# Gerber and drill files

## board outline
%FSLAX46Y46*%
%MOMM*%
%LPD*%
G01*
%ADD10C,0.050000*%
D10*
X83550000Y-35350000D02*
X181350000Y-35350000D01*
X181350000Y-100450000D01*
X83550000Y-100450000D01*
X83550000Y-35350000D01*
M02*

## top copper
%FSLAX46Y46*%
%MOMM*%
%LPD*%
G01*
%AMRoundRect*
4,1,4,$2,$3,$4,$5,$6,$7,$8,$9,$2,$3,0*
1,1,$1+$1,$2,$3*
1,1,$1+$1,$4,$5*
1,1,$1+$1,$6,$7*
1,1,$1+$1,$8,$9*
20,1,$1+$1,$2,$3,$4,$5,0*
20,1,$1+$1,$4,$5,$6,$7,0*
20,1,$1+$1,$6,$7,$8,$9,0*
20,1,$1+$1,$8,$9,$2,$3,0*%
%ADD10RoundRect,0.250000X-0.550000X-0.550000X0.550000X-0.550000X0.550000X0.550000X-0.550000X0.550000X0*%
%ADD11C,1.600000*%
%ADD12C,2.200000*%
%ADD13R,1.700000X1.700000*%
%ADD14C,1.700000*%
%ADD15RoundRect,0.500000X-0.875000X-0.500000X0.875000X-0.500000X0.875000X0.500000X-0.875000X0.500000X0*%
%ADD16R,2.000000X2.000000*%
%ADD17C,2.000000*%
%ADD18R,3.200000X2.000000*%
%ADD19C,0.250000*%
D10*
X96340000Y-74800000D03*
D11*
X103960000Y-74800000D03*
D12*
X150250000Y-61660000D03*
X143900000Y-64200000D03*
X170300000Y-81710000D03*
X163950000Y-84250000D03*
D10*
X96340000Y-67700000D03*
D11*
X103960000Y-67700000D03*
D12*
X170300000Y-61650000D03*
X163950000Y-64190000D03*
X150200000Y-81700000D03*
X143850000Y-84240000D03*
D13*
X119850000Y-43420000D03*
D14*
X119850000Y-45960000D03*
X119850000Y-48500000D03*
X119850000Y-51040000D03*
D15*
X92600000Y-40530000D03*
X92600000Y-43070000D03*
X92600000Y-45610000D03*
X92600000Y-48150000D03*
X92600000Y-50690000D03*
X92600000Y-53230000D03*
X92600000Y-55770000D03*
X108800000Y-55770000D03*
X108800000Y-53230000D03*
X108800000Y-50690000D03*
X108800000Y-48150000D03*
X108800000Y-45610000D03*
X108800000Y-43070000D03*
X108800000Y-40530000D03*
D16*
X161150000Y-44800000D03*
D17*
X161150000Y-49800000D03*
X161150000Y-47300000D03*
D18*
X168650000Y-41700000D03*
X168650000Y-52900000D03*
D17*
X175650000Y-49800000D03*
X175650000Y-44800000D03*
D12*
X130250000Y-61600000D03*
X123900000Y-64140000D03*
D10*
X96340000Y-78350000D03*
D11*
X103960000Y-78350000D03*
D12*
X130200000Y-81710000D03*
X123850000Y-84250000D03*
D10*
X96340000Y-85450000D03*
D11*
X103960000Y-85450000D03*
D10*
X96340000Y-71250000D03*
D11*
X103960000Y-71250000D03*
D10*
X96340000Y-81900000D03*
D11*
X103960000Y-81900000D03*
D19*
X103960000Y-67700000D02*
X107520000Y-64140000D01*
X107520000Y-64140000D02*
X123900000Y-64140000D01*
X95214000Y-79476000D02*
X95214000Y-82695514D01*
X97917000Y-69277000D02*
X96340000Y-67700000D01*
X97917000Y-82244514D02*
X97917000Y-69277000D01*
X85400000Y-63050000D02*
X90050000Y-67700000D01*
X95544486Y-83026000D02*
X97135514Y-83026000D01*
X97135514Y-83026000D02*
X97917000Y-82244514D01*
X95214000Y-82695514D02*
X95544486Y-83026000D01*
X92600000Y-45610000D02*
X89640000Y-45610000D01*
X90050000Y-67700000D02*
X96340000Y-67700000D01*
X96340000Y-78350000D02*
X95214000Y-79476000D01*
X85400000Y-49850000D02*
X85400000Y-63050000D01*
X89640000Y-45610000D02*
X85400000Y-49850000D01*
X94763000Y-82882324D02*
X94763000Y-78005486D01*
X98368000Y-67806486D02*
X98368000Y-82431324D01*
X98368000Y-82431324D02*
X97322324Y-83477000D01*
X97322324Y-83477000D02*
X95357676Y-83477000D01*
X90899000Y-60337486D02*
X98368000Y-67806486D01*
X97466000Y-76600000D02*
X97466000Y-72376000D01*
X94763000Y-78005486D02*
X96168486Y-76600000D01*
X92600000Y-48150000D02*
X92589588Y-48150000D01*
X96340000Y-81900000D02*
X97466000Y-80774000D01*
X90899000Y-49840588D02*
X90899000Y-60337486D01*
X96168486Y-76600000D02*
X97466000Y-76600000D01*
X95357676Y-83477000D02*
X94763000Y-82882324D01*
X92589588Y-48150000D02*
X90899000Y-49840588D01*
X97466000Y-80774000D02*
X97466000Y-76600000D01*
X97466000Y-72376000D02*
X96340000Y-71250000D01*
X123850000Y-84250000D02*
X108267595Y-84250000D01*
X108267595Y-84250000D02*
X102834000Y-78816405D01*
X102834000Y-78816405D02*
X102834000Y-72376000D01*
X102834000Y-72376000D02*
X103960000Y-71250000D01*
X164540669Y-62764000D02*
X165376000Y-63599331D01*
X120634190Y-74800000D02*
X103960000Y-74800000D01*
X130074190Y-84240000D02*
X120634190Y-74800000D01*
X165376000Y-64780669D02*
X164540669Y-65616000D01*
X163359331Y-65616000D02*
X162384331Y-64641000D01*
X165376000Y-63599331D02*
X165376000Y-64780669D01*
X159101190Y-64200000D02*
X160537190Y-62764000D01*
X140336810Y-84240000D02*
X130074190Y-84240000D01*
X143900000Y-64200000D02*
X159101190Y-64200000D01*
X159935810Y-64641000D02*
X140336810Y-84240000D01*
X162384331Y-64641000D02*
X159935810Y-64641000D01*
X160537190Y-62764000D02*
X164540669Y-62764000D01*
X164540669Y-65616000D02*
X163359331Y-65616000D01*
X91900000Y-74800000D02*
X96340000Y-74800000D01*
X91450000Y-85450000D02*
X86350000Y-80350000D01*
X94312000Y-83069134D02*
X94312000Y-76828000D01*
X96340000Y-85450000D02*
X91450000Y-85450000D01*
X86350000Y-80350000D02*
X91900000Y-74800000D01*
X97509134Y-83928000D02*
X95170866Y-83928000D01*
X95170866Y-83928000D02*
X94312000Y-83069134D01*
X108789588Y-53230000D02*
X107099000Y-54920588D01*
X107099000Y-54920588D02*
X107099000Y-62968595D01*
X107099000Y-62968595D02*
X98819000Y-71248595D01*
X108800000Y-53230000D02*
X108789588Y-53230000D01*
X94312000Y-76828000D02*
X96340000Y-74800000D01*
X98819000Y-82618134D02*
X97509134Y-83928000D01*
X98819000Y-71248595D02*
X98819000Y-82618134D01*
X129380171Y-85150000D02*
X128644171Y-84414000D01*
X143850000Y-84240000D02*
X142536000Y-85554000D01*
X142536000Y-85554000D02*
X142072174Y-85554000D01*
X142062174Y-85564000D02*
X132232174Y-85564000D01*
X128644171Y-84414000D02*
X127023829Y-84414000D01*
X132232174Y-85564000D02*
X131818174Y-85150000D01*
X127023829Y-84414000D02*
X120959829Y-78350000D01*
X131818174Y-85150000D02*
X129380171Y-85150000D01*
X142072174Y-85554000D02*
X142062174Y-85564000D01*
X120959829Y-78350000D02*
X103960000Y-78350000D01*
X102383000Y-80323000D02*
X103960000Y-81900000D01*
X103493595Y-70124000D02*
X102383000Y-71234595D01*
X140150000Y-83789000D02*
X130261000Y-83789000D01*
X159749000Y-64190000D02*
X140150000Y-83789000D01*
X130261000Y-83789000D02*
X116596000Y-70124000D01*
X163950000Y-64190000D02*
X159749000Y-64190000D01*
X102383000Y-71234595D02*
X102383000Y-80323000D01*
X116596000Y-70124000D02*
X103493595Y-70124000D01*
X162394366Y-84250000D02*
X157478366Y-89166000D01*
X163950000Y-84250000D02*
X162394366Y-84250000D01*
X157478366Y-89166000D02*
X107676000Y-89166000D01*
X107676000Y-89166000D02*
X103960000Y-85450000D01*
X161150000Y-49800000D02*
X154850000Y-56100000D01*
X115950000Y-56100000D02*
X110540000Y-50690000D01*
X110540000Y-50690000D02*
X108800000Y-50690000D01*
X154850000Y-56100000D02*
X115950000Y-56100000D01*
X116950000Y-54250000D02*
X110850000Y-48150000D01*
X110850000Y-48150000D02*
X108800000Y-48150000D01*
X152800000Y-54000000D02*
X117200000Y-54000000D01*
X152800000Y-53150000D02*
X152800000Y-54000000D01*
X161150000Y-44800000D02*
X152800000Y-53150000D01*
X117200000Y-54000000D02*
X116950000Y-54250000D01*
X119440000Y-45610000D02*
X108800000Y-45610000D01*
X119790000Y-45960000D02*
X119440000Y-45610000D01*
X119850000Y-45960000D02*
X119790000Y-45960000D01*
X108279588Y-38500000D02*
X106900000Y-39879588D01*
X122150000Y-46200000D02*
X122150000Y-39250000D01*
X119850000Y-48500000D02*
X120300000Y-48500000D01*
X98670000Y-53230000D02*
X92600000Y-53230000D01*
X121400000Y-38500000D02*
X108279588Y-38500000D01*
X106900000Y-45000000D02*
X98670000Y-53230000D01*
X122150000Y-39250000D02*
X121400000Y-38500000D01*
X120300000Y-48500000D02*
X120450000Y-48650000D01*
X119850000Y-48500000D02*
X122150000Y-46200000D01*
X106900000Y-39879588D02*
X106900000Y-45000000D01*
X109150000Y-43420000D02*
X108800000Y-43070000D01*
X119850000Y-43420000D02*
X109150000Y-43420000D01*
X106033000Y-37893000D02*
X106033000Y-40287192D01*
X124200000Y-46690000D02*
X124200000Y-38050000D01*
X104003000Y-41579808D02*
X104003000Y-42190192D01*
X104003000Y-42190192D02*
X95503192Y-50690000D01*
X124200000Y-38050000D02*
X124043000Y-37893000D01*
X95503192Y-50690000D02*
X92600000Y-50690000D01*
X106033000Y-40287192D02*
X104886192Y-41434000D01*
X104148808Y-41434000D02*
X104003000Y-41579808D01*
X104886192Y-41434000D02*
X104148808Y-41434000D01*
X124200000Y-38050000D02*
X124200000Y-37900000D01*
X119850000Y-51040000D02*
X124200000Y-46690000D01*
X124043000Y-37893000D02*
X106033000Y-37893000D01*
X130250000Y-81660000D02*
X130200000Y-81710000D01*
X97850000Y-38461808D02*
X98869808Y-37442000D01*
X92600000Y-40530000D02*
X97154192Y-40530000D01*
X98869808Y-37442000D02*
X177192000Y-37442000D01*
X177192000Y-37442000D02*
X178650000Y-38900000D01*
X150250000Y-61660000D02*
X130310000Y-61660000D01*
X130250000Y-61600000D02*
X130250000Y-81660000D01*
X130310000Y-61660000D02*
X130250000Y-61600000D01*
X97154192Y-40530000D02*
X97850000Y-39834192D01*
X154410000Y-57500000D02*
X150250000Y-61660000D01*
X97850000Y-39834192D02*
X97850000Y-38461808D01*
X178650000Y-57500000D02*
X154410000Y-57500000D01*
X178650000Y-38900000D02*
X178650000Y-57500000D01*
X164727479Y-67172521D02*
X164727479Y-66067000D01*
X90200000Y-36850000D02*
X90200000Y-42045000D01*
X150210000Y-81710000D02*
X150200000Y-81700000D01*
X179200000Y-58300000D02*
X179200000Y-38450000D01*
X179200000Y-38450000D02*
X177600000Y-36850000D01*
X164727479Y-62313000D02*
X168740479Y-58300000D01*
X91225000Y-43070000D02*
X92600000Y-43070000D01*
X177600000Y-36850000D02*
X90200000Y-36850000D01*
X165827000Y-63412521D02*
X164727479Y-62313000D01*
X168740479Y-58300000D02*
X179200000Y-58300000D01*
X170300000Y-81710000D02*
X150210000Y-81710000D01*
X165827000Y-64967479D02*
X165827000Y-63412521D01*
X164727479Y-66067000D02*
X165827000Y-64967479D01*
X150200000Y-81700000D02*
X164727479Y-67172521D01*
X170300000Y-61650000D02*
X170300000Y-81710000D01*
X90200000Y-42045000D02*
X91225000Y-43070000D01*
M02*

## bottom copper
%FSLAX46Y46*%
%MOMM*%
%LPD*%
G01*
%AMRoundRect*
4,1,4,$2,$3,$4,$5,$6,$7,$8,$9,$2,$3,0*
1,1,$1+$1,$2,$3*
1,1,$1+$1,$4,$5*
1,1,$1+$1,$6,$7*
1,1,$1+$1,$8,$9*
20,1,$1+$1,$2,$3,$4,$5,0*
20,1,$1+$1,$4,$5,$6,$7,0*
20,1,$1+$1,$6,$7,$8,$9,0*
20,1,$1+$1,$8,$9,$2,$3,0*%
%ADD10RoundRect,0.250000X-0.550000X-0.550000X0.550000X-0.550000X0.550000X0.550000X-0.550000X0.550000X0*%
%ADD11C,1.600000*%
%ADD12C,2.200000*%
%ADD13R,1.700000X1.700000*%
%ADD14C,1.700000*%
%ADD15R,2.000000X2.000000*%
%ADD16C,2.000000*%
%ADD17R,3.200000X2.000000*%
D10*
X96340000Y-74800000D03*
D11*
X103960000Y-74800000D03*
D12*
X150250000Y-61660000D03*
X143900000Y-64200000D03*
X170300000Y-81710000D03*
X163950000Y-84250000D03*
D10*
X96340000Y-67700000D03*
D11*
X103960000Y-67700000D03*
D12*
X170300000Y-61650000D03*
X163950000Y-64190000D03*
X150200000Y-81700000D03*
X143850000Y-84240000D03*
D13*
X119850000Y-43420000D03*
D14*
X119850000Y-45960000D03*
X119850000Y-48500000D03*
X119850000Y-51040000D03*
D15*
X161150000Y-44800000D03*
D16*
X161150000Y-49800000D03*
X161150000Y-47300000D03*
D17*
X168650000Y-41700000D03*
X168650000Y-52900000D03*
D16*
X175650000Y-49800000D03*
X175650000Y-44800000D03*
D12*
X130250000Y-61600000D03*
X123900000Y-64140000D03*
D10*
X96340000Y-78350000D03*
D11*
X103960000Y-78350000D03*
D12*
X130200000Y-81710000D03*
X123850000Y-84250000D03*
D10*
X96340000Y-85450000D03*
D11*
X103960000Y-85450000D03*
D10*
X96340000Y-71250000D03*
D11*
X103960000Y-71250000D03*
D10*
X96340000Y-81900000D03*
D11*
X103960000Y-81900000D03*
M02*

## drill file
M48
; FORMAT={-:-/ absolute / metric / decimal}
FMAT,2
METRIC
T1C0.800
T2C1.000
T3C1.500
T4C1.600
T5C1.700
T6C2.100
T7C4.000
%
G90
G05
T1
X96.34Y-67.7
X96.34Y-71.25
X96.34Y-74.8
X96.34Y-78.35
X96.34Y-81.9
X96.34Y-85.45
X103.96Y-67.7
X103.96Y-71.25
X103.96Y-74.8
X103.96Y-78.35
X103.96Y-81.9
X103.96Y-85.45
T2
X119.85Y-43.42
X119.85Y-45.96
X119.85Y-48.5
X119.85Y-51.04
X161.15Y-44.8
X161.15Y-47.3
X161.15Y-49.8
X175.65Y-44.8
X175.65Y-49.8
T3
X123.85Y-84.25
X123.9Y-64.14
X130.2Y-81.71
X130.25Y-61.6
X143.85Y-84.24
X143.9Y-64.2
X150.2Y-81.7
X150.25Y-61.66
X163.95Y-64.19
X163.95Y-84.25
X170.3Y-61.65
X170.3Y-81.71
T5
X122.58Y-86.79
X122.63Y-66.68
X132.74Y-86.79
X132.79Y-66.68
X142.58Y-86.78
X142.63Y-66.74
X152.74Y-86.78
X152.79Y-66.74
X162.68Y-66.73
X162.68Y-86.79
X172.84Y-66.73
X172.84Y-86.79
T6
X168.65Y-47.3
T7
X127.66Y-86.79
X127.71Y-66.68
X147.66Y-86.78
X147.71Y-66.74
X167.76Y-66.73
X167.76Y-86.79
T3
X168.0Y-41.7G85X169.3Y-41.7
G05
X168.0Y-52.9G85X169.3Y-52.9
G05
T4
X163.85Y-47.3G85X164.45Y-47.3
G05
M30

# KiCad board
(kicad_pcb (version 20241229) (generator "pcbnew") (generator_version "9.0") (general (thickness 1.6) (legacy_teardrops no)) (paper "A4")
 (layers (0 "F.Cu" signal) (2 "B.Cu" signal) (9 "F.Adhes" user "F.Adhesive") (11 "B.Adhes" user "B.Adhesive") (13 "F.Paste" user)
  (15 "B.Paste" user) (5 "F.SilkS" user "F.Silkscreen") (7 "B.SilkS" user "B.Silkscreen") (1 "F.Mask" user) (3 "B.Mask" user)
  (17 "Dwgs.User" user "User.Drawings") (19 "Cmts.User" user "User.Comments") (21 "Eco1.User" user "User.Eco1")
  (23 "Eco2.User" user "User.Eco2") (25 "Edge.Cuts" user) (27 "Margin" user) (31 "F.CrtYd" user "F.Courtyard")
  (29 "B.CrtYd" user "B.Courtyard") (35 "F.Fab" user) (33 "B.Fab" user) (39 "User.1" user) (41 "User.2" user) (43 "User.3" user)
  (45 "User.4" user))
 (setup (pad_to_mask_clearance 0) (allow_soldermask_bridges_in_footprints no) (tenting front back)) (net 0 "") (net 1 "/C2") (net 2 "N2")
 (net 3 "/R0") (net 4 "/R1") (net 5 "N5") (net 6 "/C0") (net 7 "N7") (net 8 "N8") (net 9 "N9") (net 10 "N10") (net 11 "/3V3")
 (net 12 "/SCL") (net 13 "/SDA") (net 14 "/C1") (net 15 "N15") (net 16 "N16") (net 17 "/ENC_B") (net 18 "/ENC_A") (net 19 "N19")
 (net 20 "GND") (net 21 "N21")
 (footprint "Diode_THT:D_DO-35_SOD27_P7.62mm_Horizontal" (layer "F.Cu") (at 96.34 74.8)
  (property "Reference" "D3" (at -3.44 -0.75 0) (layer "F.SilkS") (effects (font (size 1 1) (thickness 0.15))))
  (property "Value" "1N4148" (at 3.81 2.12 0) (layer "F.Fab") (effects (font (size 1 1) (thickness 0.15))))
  (pad "1" thru_hole roundrect (at 0 0) (size 1.6 1.6) (drill 0.8) (layers "*.Cu" "*.Mask") (remove_unused_layers no)
   (roundrect_rratio 0.15625) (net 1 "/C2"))
  (pad "2" thru_hole circle (at 7.62 0) (size 1.6 1.6) (drill 0.8) (layers "*.Cu" "*.Mask") (remove_unused_layers no) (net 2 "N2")))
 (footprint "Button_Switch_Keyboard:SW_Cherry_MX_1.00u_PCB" (layer "F.Cu") (at 150.25 61.66)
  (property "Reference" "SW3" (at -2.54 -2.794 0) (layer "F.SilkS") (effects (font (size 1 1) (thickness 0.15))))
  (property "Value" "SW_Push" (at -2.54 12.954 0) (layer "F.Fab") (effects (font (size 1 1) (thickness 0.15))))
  (pad "" np_thru_hole circle (at -7.62 5.08) (size 1.7 1.7) (drill 1.7) (layers "*.Cu" "*.Mask"))
  (pad "" np_thru_hole circle (at -2.54 5.08) (size 4 4) (drill 4) (layers "*.Cu" "*.Mask"))
  (pad "" np_thru_hole circle (at 2.54 5.08) (size 1.7 1.7) (drill 1.7) (layers "*.Cu" "*.Mask"))
  (pad "1" thru_hole circle (at 0 0) (size 2.2 2.2) (drill 1.5) (layers "*.Cu" "*.Mask") (remove_unused_layers no) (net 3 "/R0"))
  (pad "2" thru_hole circle (at -6.35 2.54) (size 2.2 2.2) (drill 1.5) (layers "*.Cu" "*.Mask") (remove_unused_layers no) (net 2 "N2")))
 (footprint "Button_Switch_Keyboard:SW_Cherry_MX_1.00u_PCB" (layer "F.Cu") (at 170.3 81.71)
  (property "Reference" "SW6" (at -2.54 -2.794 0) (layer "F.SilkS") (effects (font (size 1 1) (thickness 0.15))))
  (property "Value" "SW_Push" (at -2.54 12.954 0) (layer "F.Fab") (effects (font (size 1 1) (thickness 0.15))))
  (pad "" np_thru_hole circle (at -7.62 5.08) (size 1.7 1.7) (drill 1.7) (layers "*.Cu" "*.Mask"))
  (pad "" np_thru_hole circle (at -2.54 5.08) (size 4 4) (drill 4) (layers "*.Cu" "*.Mask"))
  (pad "" np_thru_hole circle (at 2.54 5.08) (size 1.7 1.7) (drill 1.7) (layers "*.Cu" "*.Mask"))
  (pad "1" thru_hole circle (at 0 0) (size 2.2 2.2) (drill 1.5) (layers "*.Cu" "*.Mask") (remove_unused_layers no) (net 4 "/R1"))
  (pad "2" thru_hole circle (at -6.35 2.54) (size 2.2 2.2) (drill 1.5) (layers "*.Cu" "*.Mask") (remove_unused_layers no) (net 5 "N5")))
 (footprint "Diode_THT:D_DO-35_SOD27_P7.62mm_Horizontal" (layer "F.Cu") (at 96.34 67.7)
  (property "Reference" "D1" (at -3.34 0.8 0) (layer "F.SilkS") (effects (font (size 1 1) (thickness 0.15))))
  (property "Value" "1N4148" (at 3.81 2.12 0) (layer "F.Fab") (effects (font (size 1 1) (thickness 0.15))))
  (pad "1" thru_hole roundrect (at 0 0) (size 1.6 1.6) (drill 0.8) (layers "*.Cu" "*.Mask") (remove_unused_layers no)
   (roundrect_rratio 0.15625) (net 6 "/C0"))
  (pad "2" thru_hole circle (at 7.62 0) (size 1.6 1.6) (drill 0.8) (layers "*.Cu" "*.Mask") (remove_unused_layers no) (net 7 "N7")))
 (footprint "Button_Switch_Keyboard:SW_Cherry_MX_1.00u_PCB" (layer "F.Cu") (at 170.3 61.65)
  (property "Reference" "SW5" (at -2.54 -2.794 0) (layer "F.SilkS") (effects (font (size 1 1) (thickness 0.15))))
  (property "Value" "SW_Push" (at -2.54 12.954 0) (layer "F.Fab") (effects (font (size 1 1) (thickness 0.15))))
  (pad "" np_thru_hole circle (at -7.62 5.08) (size 1.7 1.7) (drill 1.7) (layers "*.Cu" "*.Mask"))
  (pad "" np_thru_hole circle (at -2.54 5.08) (size 4 4) (drill 4) (layers "*.Cu" "*.Mask"))
  (pad "" np_thru_hole circle (at 2.54 5.08) (size 1.7 1.7) (drill 1.7) (layers "*.Cu" "*.Mask"))
  (pad "1" thru_hole circle (at 0 0) (size 2.2 2.2) (drill 1.5) (layers "*.Cu" "*.Mask") (remove_unused_layers no) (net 4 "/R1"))
  (pad "2" thru_hole circle (at -6.35 2.54) (size 2.2 2.2) (drill 1.5) (layers "*.Cu" "*.Mask") (remove_unused_layers no) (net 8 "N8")))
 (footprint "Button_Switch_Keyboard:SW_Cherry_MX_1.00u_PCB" (layer "F.Cu") (at 150.2 81.7)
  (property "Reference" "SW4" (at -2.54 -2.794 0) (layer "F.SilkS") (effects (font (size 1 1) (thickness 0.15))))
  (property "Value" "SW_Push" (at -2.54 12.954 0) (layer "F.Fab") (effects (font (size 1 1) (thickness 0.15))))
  (pad "" np_thru_hole circle (at -7.62 5.08) (size 1.7 1.7) (drill 1.7) (layers "*.Cu" "*.Mask"))
  (pad "" np_thru_hole circle (at -2.54 5.08) (size 4 4) (drill 4) (layers "*.Cu" "*.Mask"))
  (pad "" np_thru_hole circle (at 2.54 5.08) (size 1.7 1.7) (drill 1.7) (layers "*.Cu" "*.Mask"))
  (pad "1" thru_hole circle (at 0 0) (size 2.2 2.2) (drill 1.5) (layers "*.Cu" "*.Mask") (remove_unused_layers no) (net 4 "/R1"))
  (pad "2" thru_hole circle (at -6.35 2.54) (size 2.2 2.2) (drill 1.5) (layers "*.Cu" "*.Mask") (remove_unused_layers no) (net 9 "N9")))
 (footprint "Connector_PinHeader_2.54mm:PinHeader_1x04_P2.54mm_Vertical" (layer "F.Cu") (at 119.85 43.42)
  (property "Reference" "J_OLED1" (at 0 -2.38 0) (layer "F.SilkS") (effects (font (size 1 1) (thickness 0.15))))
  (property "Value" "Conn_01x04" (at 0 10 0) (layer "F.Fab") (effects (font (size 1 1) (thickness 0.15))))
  (pad "1" thru_hole rect (at 0 0) (size 1.7 1.7) (drill 1) (layers "*.Cu" "*.Mask") (remove_unused_layers no) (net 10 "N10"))
  (pad "2" thru_hole circle (at 0 2.54) (size 1.7 1.7) (drill 1) (layers "*.Cu" "*.Mask") (remove_unused_layers no) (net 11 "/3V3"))
  (pad "3" thru_hole circle (at 0 5.08) (size 1.7 1.7) (drill 1) (layers "*.Cu" "*.Mask") (remove_unused_layers no) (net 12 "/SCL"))
  (pad "4" thru_hole circle (at 0 7.62) (size 1.7 1.7) (drill 1) (layers "*.Cu" "*.Mask") (remove_unused_layers no) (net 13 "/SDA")))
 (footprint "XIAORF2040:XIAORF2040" (layer "F.Cu") (at 100.7 48.15)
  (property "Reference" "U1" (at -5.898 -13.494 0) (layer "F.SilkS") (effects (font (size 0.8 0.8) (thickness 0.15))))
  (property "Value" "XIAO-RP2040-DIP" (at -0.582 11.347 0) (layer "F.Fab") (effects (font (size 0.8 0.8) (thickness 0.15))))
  (pad "1" smd roundrect (at -8.1 -7.62) (size 2.75 2) (layers "F.Cu" "F.Mask" "F.Paste") (roundrect_rratio 0.25) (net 3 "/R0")
   (solder_mask_margin 0.102))
  (pad "2" smd roundrect (at -8.1 -5.08) (size 2.75 2) (layers "F.Cu" "F.Mask" "F.Paste") (roundrect_rratio 0.25) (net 4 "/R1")
   (solder_mask_margin 0.102))
  (pad "3" smd roundrect (at -8.1 -2.54) (size 2.75 2) (layers "F.Cu" "F.Mask" "F.Paste") (roundrect_rratio 0.25) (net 6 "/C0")
   (solder_mask_margin 0.102))
  (pad "4" smd roundrect (at -8.1 0) (size 2.75 2) (layers "F.Cu" "F.Mask" "F.Paste") (roundrect_rratio 0.25) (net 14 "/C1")
   (solder_mask_margin 0.102))
  (pad "5" smd roundrect (at -8.1 2.54) (size 2.75 2) (layers "F.Cu" "F.Mask" "F.Paste") (roundrect_rratio 0.25) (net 13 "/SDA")
   (solder_mask_margin 0.102))
  (pad "6" smd roundrect (at -8.1 5.08) (size 2.75 2) (layers "F.Cu" "F.Mask" "F.Paste") (roundrect_rratio 0.25) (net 12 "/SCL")
   (solder_mask_margin 0.102))
  (pad "7" smd roundrect (at -8.1 7.62) (size 2.75 2) (layers "F.Cu" "F.Mask" "F.Paste") (roundrect_rratio 0.25) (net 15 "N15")
   (solder_mask_margin 0.102))
  (pad "8" smd roundrect (at 8.1 7.62) (size 2.75 2) (layers "F.Cu" "F.Mask" "F.Paste") (roundrect_rratio 0.25) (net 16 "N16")
   (solder_mask_margin 0.102))
  (pad "9" smd roundrect (at 8.1 5.08) (size 2.75 2) (layers "F.Cu" "F.Mask" "F.Paste") (roundrect_rratio 0.25) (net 1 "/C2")
   (solder_mask_margin 0.102))
  (pad "10" smd roundrect (at 8.1 2.54) (size 2.75 2) (layers "F.Cu" "F.Mask" "F.Paste") (roundrect_rratio 0.25) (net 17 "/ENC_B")
   (solder_mask_margin 0.102))
  (pad "11" smd roundrect (at 8.1 0) (size 2.75 2) (layers "F.Cu" "F.Mask" "F.Paste") (roundrect_rratio 0.25) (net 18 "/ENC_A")
   (solder_mask_margin 0.102))
  (pad "12" smd roundrect (at 8.1 -2.54) (size 2.75 2) (layers "F.Cu" "F.Mask" "F.Paste") (roundrect_rratio 0.25) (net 11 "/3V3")
   (solder_mask_margin 0.102))
  (pad "13" smd roundrect (at 8.1 -5.08) (size 2.75 2) (layers "F.Cu" "F.Mask" "F.Paste") (roundrect_rratio 0.25) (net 10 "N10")
   (solder_mask_margin 0.102))
  (pad "14" smd roundrect (at 8.1 -7.62) (size 2.75 2) (layers "F.Cu" "F.Mask" "F.Paste") (roundrect_rratio 0.25) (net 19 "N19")
   (solder_mask_margin 0.102))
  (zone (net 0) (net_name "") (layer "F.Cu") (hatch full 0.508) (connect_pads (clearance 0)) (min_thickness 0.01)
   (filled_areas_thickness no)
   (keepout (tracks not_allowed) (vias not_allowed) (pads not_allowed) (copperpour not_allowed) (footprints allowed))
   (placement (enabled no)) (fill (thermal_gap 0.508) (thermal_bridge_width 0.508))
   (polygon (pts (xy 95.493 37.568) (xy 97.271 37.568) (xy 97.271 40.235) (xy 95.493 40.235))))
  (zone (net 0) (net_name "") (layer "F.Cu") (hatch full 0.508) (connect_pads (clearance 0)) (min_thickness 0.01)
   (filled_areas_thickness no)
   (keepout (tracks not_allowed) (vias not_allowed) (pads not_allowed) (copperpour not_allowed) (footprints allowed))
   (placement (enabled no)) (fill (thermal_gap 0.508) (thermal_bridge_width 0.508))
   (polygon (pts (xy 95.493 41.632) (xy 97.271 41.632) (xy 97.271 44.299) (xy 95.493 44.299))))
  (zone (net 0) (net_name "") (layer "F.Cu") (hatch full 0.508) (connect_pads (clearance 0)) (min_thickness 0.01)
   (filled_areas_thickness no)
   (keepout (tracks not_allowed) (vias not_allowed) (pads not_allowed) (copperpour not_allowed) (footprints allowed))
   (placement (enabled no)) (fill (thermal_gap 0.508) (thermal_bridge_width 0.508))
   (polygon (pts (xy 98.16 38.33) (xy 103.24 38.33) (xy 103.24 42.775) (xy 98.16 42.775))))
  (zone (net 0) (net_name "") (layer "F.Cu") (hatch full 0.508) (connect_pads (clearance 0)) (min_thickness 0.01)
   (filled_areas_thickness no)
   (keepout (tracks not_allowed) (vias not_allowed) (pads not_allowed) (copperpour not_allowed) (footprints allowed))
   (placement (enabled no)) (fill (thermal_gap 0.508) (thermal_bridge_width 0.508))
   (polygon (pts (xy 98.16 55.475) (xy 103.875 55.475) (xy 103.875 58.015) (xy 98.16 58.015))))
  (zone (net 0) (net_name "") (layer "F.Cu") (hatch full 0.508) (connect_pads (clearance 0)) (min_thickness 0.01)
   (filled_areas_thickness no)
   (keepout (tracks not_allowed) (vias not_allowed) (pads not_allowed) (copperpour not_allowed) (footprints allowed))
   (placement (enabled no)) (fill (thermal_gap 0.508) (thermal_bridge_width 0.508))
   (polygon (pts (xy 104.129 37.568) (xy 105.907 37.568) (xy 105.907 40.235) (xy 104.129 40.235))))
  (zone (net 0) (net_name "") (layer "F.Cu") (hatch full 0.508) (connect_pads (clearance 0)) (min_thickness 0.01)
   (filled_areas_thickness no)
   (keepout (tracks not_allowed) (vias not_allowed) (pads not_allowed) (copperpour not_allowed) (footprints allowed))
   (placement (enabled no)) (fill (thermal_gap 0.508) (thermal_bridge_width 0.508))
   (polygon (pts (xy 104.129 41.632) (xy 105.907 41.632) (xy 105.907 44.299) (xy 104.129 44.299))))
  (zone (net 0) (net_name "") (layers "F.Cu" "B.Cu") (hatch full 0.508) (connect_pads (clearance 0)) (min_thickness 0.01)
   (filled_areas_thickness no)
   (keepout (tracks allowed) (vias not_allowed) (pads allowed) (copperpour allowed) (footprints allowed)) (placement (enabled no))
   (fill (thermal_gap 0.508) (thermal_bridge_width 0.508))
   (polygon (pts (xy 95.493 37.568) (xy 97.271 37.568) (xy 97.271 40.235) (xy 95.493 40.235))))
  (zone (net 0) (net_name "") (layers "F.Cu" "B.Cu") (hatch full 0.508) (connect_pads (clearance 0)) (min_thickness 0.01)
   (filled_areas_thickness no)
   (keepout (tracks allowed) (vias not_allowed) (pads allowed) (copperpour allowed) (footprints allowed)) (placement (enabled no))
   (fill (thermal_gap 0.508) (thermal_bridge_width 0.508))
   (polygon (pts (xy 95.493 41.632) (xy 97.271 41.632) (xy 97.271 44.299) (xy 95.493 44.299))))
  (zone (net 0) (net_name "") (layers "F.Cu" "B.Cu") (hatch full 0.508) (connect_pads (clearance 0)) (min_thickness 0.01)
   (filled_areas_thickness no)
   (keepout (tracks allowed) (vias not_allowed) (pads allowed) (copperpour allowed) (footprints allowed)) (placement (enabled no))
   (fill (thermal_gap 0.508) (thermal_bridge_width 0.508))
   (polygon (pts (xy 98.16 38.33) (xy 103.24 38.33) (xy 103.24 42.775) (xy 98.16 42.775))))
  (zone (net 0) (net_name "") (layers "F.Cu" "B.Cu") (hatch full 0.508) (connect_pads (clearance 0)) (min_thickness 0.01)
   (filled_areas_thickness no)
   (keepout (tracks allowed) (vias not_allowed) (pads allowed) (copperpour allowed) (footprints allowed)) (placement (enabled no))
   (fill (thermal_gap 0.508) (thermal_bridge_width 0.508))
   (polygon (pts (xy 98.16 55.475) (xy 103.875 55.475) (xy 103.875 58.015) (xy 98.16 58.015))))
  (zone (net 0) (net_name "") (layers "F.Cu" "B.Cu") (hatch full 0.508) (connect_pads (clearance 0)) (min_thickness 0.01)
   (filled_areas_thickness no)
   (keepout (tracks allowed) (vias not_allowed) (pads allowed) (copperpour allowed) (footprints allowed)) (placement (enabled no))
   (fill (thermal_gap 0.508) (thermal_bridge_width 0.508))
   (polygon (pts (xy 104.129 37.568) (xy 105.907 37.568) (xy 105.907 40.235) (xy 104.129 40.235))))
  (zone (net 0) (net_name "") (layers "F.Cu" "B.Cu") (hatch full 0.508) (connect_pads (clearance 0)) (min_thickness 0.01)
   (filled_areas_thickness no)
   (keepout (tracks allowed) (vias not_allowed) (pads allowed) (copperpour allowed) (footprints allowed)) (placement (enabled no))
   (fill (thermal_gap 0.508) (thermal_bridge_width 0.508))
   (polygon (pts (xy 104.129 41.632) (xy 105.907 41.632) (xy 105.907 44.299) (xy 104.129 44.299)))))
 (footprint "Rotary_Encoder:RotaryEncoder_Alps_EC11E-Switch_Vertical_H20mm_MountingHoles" (layer "F.Cu") (at 161.15 44.8)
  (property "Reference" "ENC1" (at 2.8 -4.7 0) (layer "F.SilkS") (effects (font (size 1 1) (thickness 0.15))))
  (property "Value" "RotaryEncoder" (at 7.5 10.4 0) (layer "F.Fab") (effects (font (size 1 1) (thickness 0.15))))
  (pad "" np_thru_hole oval (at 3 2.5) (size 2.2 1.6) (drill oval 2.2 1.6) (layers "*.Mask"))
  (pad "" np_thru_hole circle (at 7.5 2.5) (size 2.1 2.1) (drill 2.1) (layers "*.Mask"))
  (pad "A" thru_hole rect (at 0 0) (size 2 2) (drill 1) (layers "*.Cu" "*.Mask") (remove_unused_layers no) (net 18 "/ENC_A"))
  (pad "B" thru_hole circle (at 0 5) (size 2 2) (drill 1) (layers "*.Cu" "*.Mask") (remove_unused_layers no) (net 17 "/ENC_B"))
  (pad "C" thru_hole circle (at 0 2.5) (size 2 2) (drill 1) (layers "*.Cu" "*.Mask") (remove_unused_layers no) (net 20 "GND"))
  (pad "MP" thru_hole rect (at 7.5 -3.1) (size 3.2 2) (drill oval 2.8 1.5) (layers "*.Cu" "*.Mask") (remove_unused_layers no))
  (pad "MP" thru_hole rect (at 7.5 8.1) (size 3.2 2) (drill oval 2.8 1.5) (layers "*.Cu" "*.Mask") (remove_unused_layers no))
  (pad "S1" thru_hole circle (at 14.5 5) (size 2 2) (drill 1) (layers "*.Cu" "*.Mask") (remove_unused_layers no))
  (pad "S2" thru_hole circle (at 14.5 0) (size 2 2) (drill 1) (layers "*.Cu" "*.Mask") (remove_unused_layers no)))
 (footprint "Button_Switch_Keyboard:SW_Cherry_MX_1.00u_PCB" (layer "F.Cu") (at 130.25 61.6)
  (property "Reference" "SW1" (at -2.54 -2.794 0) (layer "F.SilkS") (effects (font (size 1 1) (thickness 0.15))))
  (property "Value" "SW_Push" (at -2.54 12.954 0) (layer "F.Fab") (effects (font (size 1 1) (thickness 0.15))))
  (pad "" np_thru_hole circle (at -7.62 5.08) (size 1.7 1.7) (drill 1.7) (layers "*.Cu" "*.Mask"))
  (pad "" np_thru_hole circle (at -2.54 5.08) (size 4 4) (drill 4) (layers "*.Cu" "*.Mask"))
  (pad "" np_thru_hole circle (at 2.54 5.08) (size 1.7 1.7) (drill 1.7) (layers "*.Cu" "*.Mask"))
  (pad "1" thru_hole circle (at 0 0) (size 2.2 2.2) (drill 1.5) (layers "*.Cu" "*.Mask") (remove_unused_layers no) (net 3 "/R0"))
  (pad "2" thru_hole circle (at -6.35 2.54) (size 2.2 2.2) (drill 1.5) (layers "*.Cu" "*.Mask") (remove_unused_layers no) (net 7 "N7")))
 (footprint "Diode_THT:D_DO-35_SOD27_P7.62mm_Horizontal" (layer "F.Cu") (at 96.34 78.35)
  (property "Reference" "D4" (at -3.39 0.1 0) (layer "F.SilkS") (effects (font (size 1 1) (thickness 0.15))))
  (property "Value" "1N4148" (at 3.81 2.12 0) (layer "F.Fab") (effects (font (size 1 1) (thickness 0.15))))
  (pad "1" thru_hole roundrect (at 0 0) (size 1.6 1.6) (drill 0.8) (layers "*.Cu" "*.Mask") (remove_unused_layers no)
   (roundrect_rratio 0.15625) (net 6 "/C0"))
  (pad "2" thru_hole circle (at 7.62 0) (size 1.6 1.6) (drill 0.8) (layers "*.Cu" "*.Mask") (remove_unused_layers no) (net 9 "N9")))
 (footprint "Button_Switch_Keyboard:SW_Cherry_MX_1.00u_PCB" (layer "F.Cu") (at 130.2 81.71)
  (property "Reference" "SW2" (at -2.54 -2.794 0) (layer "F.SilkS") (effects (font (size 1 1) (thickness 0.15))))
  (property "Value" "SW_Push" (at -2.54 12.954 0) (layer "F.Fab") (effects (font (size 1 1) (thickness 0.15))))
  (pad "" np_thru_hole circle (at -7.62 5.08) (size 1.7 1.7) (drill 1.7) (layers "*.Cu" "*.Mask"))
  (pad "" np_thru_hole circle (at -2.54 5.08) (size 4 4) (drill 4) (layers "*.Cu" "*.Mask"))
  (pad "" np_thru_hole circle (at 2.54 5.08) (size 1.7 1.7) (drill 1.7) (layers "*.Cu" "*.Mask"))
  (pad "1" thru_hole circle (at 0 0) (size 2.2 2.2) (drill 1.5) (layers "*.Cu" "*.Mask") (remove_unused_layers no) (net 3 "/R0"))
  (pad "2" thru_hole circle (at -6.35 2.54) (size 2.2 2.2) (drill 1.5) (layers "*.Cu" "*.Mask") (remove_unused_layers no) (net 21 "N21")))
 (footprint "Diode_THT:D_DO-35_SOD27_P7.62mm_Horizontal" (layer "F.Cu") (at 96.34 85.45)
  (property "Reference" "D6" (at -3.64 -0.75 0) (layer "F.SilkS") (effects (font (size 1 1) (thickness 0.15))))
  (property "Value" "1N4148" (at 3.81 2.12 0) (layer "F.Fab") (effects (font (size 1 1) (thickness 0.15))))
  (pad "1" thru_hole roundrect (at 0 0) (size 1.6 1.6) (drill 0.8) (layers "*.Cu" "*.Mask") (remove_unused_layers no)
   (roundrect_rratio 0.15625) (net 1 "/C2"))
  (pad "2" thru_hole circle (at 7.62 0) (size 1.6 1.6) (drill 0.8) (layers "*.Cu" "*.Mask") (remove_unused_layers no) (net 5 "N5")))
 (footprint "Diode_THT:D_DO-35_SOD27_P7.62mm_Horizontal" (layer "F.Cu") (at 96.34 71.25)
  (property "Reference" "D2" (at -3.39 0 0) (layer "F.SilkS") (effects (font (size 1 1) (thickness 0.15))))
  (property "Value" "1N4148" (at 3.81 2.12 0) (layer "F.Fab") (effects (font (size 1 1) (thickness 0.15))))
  (pad "1" thru_hole roundrect (at 0 0) (size 1.6 1.6) (drill 0.8) (layers "*.Cu" "*.Mask") (remove_unused_layers no)
   (roundrect_rratio 0.15625) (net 14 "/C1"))
  (pad "2" thru_hole circle (at 7.62 0) (size 1.6 1.6) (drill 0.8) (layers "*.Cu" "*.Mask") (remove_unused_layers no) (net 21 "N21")))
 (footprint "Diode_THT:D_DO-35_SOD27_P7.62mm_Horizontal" (layer "F.Cu") (at 96.34 81.9)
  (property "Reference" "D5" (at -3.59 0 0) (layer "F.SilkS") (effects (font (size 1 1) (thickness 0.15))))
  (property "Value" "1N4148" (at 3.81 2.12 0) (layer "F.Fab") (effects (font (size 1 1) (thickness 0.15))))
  (pad "1" thru_hole roundrect (at 0 0) (size 1.6 1.6) (drill 0.8) (layers "*.Cu" "*.Mask") (remove_unused_layers no)
   (roundrect_rratio 0.15625) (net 14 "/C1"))
  (pad "2" thru_hole circle (at 7.62 0) (size 1.6 1.6) (drill 0.8) (layers "*.Cu" "*.Mask") (remove_unused_layers no) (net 8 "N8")))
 (gr_rect (start 83.55 35.35) (end 181.35 100.45) (stroke (width 0.05) (type default)) (fill no) (layer "Edge.Cuts"))
 (segment (start 103.96 67.7) (end 107.52 64.14) (width 0.25) (layer "F.Cu") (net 7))
 (segment (start 107.52 64.14) (end 123.9 64.14) (width 0.25) (layer "F.Cu") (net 7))
 (segment (start 95.214 79.476) (end 95.214 82.695514) (width 0.25) (layer "F.Cu") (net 6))
 (segment (start 97.917 69.277) (end 96.34 67.7) (width 0.25) (layer "F.Cu") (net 6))
 (segment (start 97.917 82.244514) (end 97.917 69.277) (width 0.25) (layer "F.Cu") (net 6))
 (segment (start 85.4 63.05) (end 90.05 67.7) (width 0.25) (layer "F.Cu") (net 6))
 (segment (start 95.544486 83.026) (end 97.135514 83.026) (width 0.25) (layer "F.Cu") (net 6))
 (segment (start 97.135514 83.026) (end 97.917 82.244514) (width 0.25) (layer "F.Cu") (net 6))
 (segment (start 95.214 82.695514) (end 95.544486 83.026) (width 0.25) (layer "F.Cu") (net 6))
 (segment (start 92.6 45.61) (end 89.64 45.61) (width 0.25) (layer "F.Cu") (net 6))
 (segment (start 90.05 67.7) (end 96.34 67.7) (width 0.25) (layer "F.Cu") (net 6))
 (segment (start 96.34 78.35) (end 95.214 79.476) (width 0.25) (layer "F.Cu") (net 6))
 (segment (start 85.4 49.85) (end 85.4 63.05) (width 0.25) (layer "F.Cu") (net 6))
 (segment (start 89.64 45.61) (end 85.4 49.85) (width 0.25) (layer "F.Cu") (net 6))
 (segment (start 94.763 82.882324) (end 94.763 78.005486) (width 0.25) (layer "F.Cu") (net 14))
 (segment (start 98.368 67.806486) (end 98.368 82.431324) (width 0.25) (layer "F.Cu") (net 14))
 (segment (start 98.368 82.431324) (end 97.322324 83.477) (width 0.25) (layer "F.Cu") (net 14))
 (segment (start 97.322324 83.477) (end 95.357676 83.477) (width 0.25) (layer "F.Cu") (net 14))
 (segment (start 90.899 60.337486) (end 98.368 67.806486) (width 0.25) (layer "F.Cu") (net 14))
 (segment (start 97.466 76.6) (end 97.466 72.376) (width 0.25) (layer "F.Cu") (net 14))
 (segment (start 94.763 78.005486) (end 96.168486 76.6) (width 0.25) (layer "F.Cu") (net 14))
 (segment (start 92.6 48.15) (end 92.589588 48.15) (width 0.25) (layer "F.Cu") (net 14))
 (segment (start 96.34 81.9) (end 97.466 80.774) (width 0.25) (layer "F.Cu") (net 14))
 (segment (start 90.899 49.840588) (end 90.899 60.337486) (width 0.25) (layer "F.Cu") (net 14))
 (segment (start 96.168486 76.6) (end 97.466 76.6) (width 0.25) (layer "F.Cu") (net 14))
 (segment (start 95.357676 83.477) (end 94.763 82.882324) (width 0.25) (layer "F.Cu") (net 14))
 (segment (start 92.589588 48.15) (end 90.899 49.840588) (width 0.25) (layer "F.Cu") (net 14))
 (segment (start 97.466 80.774) (end 97.466 76.6) (width 0.25) (layer "F.Cu") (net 14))
 (segment (start 97.466 72.376) (end 96.34 71.25) (width 0.25) (layer "F.Cu") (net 14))
 (segment (start 123.85 84.25) (end 108.267595 84.25) (width 0.25) (layer "F.Cu") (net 21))
 (segment (start 108.267595 84.25) (end 102.834 78.816405) (width 0.25) (layer "F.Cu") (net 21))
 (segment (start 102.834 78.816405) (end 102.834 72.376) (width 0.25) (layer "F.Cu") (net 21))
 (segment (start 102.834 72.376) (end 103.96 71.25) (width 0.25) (layer "F.Cu") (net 21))
 (segment (start 164.540669 62.764) (end 165.376 63.599331) (width 0.25) (layer "F.Cu") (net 2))
 (segment (start 120.63419 74.8) (end 103.96 74.8) (width 0.25) (layer "F.Cu") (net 2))
 (segment (start 130.07419 84.24) (end 120.63419 74.8) (width 0.25) (layer "F.Cu") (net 2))
 (segment (start 165.376 64.780669) (end 164.540669 65.616) (width 0.25) (layer "F.Cu") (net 2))
 (segment (start 163.359331 65.616) (end 162.384331 64.641) (width 0.25) (layer "F.Cu") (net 2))
 (segment (start 165.376 63.599331) (end 165.376 64.780669) (width 0.25) (layer "F.Cu") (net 2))
 (segment (start 159.10119 64.2) (end 160.53719 62.764) (width 0.25) (layer "F.Cu") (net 2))
 (segment (start 140.33681 84.24) (end 130.07419 84.24) (width 0.25) (layer "F.Cu") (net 2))
 (segment (start 143.9 64.2) (end 159.10119 64.2) (width 0.25) (layer "F.Cu") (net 2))
 (segment (start 159.93581 64.641) (end 140.33681 84.24) (width 0.25) (layer "F.Cu") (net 2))
 (segment (start 162.384331 64.641) (end 159.93581 64.641) (width 0.25) (layer "F.Cu") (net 2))
 (segment (start 160.53719 62.764) (end 164.540669 62.764) (width 0.25) (layer "F.Cu") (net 2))
 (segment (start 164.540669 65.616) (end 163.359331 65.616) (width 0.25) (layer "F.Cu") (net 2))
 (segment (start 91.9 74.8) (end 96.34 74.8) (width 0.25) (layer "F.Cu") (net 1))
 (segment (start 91.45 85.45) (end 86.35 80.35) (width 0.25) (layer "F.Cu") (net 1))
 (segment (start 94.312 83.069134) (end 94.312 76.828) (width 0.25) (layer "F.Cu") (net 1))
 (segment (start 96.34 85.45) (end 91.45 85.45) (width 0.25) (layer "F.Cu") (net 1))
 (segment (start 86.35 80.35) (end 91.9 74.8) (width 0.25) (layer "F.Cu") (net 1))
 (segment (start 97.509134 83.928) (end 95.170866 83.928) (width 0.25) (layer "F.Cu") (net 1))
 (segment (start 95.170866 83.928) (end 94.312 83.069134) (width 0.25) (layer "F.Cu") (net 1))
 (segment (start 108.789588 53.23) (end 107.099 54.920588) (width 0.25) (layer "F.Cu") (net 1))
 (segment (start 107.099 54.920588) (end 107.099 62.968595) (width 0.25) (layer "F.Cu") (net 1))
 (segment (start 107.099 62.968595) (end 98.819 71.248595) (width 0.25) (layer "F.Cu") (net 1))
 (segment (start 108.8 53.23) (end 108.789588 53.23) (width 0.25) (layer "F.Cu") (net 1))
 (segment (start 94.312 76.828) (end 96.34 74.8) (width 0.25) (layer "F.Cu") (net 1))
 (segment (start 98.819 82.618134) (end 97.509134 83.928) (width 0.25) (layer "F.Cu") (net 1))
 (segment (start 98.819 71.248595) (end 98.819 82.618134) (width 0.25) (layer "F.Cu") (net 1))
 (segment (start 129.380171 85.15) (end 128.644171 84.414) (width 0.25) (layer "F.Cu") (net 9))
 (segment (start 143.85 84.24) (end 142.536 85.554) (width 0.25) (layer "F.Cu") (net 9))
 (segment (start 142.536 85.554) (end 142.072174 85.554) (width 0.25) (layer "F.Cu") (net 9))
 (segment (start 142.062174 85.564) (end 132.232174 85.564) (width 0.25) (layer "F.Cu") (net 9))
 (segment (start 128.644171 84.414) (end 127.023829 84.414) (width 0.25) (layer "F.Cu") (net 9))
 (segment (start 132.232174 85.564) (end 131.818174 85.15) (width 0.25) (layer "F.Cu") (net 9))
 (segment (start 127.023829 84.414) (end 120.959829 78.35) (width 0.25) (layer "F.Cu") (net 9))
 (segment (start 131.818174 85.15) (end 129.380171 85.15) (width 0.25) (layer "F.Cu") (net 9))
 (segment (start 142.072174 85.554) (end 142.062174 85.564) (width 0.25) (layer "F.Cu") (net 9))
 (segment (start 120.959829 78.35) (end 103.96 78.35) (width 0.25) (layer "F.Cu") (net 9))
 (segment (start 102.383 80.323) (end 103.96 81.9) (width 0.25) (layer "F.Cu") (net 8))
 (segment (start 103.493595 70.124) (end 102.383 71.234595) (width 0.25) (layer "F.Cu") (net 8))
 (segment (start 140.15 83.789) (end 130.261 83.789) (width 0.25) (layer "F.Cu") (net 8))
 (segment (start 159.749 64.19) (end 140.15 83.789) (width 0.25) (layer "F.Cu") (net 8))
 (segment (start 130.261 83.789) (end 116.596 70.124) (width 0.25) (layer "F.Cu") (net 8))
 (segment (start 163.95 64.19) (end 159.749 64.19) (width 0.25) (layer "F.Cu") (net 8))
 (segment (start 102.383 71.234595) (end 102.383 80.323) (width 0.25) (layer "F.Cu") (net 8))
 (segment (start 116.596 70.124) (end 103.493595 70.124) (width 0.25) (layer "F.Cu") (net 8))
 (segment (start 162.394366 84.25) (end 157.478366 89.166) (width 0.25) (layer "F.Cu") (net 5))
 (segment (start 163.95 84.25) (end 162.394366 84.25) (width 0.25) (layer "F.Cu") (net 5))
 (segment (start 157.478366 89.166) (end 107.676 89.166) (width 0.25) (layer "F.Cu") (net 5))
 (segment (start 107.676 89.166) (end 103.96 85.45) (width 0.25) (layer "F.Cu") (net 5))
 (segment (start 161.15 49.8) (end 154.85 56.1) (width 0.25) (layer "F.Cu") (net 17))
 (segment (start 115.95 56.1) (end 110.54 50.69) (width 0.25) (layer "F.Cu") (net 17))
 (segment (start 110.54 50.69) (end 108.8 50.69) (width 0.25) (layer "F.Cu") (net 17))
 (segment (start 154.85 56.1) (end 115.95 56.1) (width 0.25) (layer "F.Cu") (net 17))
 (segment (start 116.95 54.25) (end 110.85 48.15) (width 0.25) (layer "F.Cu") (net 18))
 (segment (start 110.85 48.15) (end 108.8 48.15) (width 0.25) (layer "F.Cu") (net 18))
 (segment (start 152.8 54) (end 117.2 54) (width 0.25) (layer "F.Cu") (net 18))
 (segment (start 152.8 53.15) (end 152.8 54) (width 0.25) (layer "F.Cu") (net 18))
 (segment (start 161.15 44.8) (end 152.8 53.15) (width 0.25) (layer "F.Cu") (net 18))
 (segment (start 117.2 54) (end 116.95 54.25) (width 0.25) (layer "F.Cu") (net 18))
 (segment (start 119.44 45.61) (end 108.8 45.61) (width 0.25) (layer "F.Cu") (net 11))
 (segment (start 119.79 45.96) (end 119.44 45.61) (width 0.25) (layer "F.Cu") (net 11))
 (segment (start 119.85 45.96) (end 119.79 45.96) (width 0.25) (layer "F.Cu") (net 11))
 (segment (start 108.279588 38.5) (end 106.9 39.879588) (width 0.25) (layer "F.Cu") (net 12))
 (segment (start 122.15 46.2) (end 122.15 39.25) (width 0.25) (layer "F.Cu") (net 12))
 (segment (start 119.85 48.5) (end 120.3 48.5) (width 0.25) (layer "F.Cu") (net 12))
 (segment (start 98.67 53.23) (end 92.6 53.23) (width 0.25) (layer "F.Cu") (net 12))
 (segment (start 121.4 38.5) (end 108.279588 38.5) (width 0.25) (layer "F.Cu") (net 12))
 (segment (start 106.9 45) (end 98.67 53.23) (width 0.25) (layer "F.Cu") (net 12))
 (segment (start 122.15 39.25) (end 121.4 38.5) (width 0.25) (layer "F.Cu") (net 12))
 (segment (start 120.3 48.5) (end 120.45 48.65) (width 0.25) (layer "F.Cu") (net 12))
 (segment (start 119.85 48.5) (end 122.15 46.2) (width 0.25) (layer "F.Cu") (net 12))
 (segment (start 106.9 39.879588) (end 106.9 45) (width 0.25) (layer "F.Cu") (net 12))
 (segment (start 109.15 43.42) (end 108.8 43.07) (width 0.25) (layer "F.Cu") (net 10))
 (segment (start 119.85 43.42) (end 109.15 43.42) (width 0.25) (layer "F.Cu") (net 10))
 (segment (start 106.033 37.893) (end 106.033 40.287192) (width 0.25) (layer "F.Cu") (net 13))
 (segment (start 124.2 46.69) (end 124.2 38.05) (width 0.25) (layer "F.Cu") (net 13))
 (segment (start 104.003 41.579808) (end 104.003 42.190192) (width 0.25) (layer "F.Cu") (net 13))
 (segment (start 104.003 42.190192) (end 95.503192 50.69) (width 0.25) (layer "F.Cu") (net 13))
 (segment (start 124.2 38.05) (end 124.043 37.893) (width 0.25) (layer "F.Cu") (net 13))
 (segment (start 95.503192 50.69) (end 92.6 50.69) (width 0.25) (layer "F.Cu") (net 13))
 (segment (start 106.033 40.287192) (end 104.886192 41.434) (width 0.25) (layer "F.Cu") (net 13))
 (segment (start 104.148808 41.434) (end 104.003 41.579808) (width 0.25) (layer "F.Cu") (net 13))
 (segment (start 104.886192 41.434) (end 104.148808 41.434) (width 0.25) (layer "F.Cu") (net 13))
 (segment (start 124.2 38.05) (end 124.2 37.9) (width 0.25) (layer "F.Cu") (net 13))
 (segment (start 119.85 51.04) (end 124.2 46.69) (width 0.25) (layer "F.Cu") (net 13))
 (segment (start 124.043 37.893) (end 106.033 37.893) (width 0.25) (layer "F.Cu") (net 13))
 (segment (start 130.25 81.66) (end 130.2 81.71) (width 0.25) (layer "F.Cu") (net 3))
 (segment (start 97.85 38.461808) (end 98.869808 37.442) (width 0.25) (layer "F.Cu") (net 3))
 (segment (start 92.6 40.53) (end 97.154192 40.53) (width 0.25) (layer "F.Cu") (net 3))
 (segment (start 98.869808 37.442) (end 177.192 37.442) (width 0.25) (layer "F.Cu") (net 3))
 (segment (start 177.192 37.442) (end 178.65 38.9) (width 0.25) (layer "F.Cu") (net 3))
 (segment (start 150.25 61.66) (end 130.31 61.66) (width 0.25) (layer "F.Cu") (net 3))
 (segment (start 130.25 61.6) (end 130.25 81.66) (width 0.25) (layer "F.Cu") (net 3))
 (segment (start 130.31 61.66) (end 130.25 61.6) (width 0.25) (layer "F.Cu") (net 3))
 (segment (start 97.154192 40.53) (end 97.85 39.834192) (width 0.25) (layer "F.Cu") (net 3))
 (segment (start 154.41 57.5) (end 150.25 61.66) (width 0.25) (layer "F.Cu") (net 3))
 (segment (start 97.85 39.834192) (end 97.85 38.461808) (width 0.25) (layer "F.Cu") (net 3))
 (segment (start 178.65 57.5) (end 154.41 57.5) (width 0.25) (layer "F.Cu") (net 3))
 (segment (start 178.65 38.9) (end 178.65 57.5) (width 0.25) (layer "F.Cu") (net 3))
 (segment (start 164.727479 67.172521) (end 164.727479 66.067) (width 0.25) (layer "F.Cu") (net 4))
 (segment (start 90.2 36.85) (end 90.2 42.045) (width 0.25) (layer "F.Cu") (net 4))
 (segment (start 150.21 81.71) (end 150.2 81.7) (width 0.25) (layer "F.Cu") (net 4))
 (segment (start 179.2 58.3) (end 179.2 38.45) (width 0.25) (layer "F.Cu") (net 4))
 (segment (start 179.2 38.45) (end 177.6 36.85) (width 0.25) (layer "F.Cu") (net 4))
 (segment (start 164.727479 62.313) (end 168.740479 58.3) (width 0.25) (layer "F.Cu") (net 4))
 (segment (start 91.225 43.07) (end 92.6 43.07) (width 0.25) (layer "F.Cu") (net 4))
 (segment (start 177.6 36.85) (end 90.2 36.85) (width 0.25) (layer "F.Cu") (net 4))
 (segment (start 165.827 63.412521) (end 164.727479 62.313) (width 0.25) (layer "F.Cu") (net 4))
 (segment (start 168.740479 58.3) (end 179.2 58.3) (width 0.25) (layer "F.Cu") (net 4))
 (segment (start 170.3 81.71) (end 150.21 81.71) (width 0.25) (layer "F.Cu") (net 4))
 (segment (start 165.827 64.967479) (end 165.827 63.412521) (width 0.25) (layer "F.Cu") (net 4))
 (segment (start 164.727479 66.067) (end 165.827 64.967479) (width 0.25) (layer "F.Cu") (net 4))
 (segment (start 150.2 81.7) (end 164.727479 67.172521) (width 0.25) (layer "F.Cu") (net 4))
 (segment (start 170.3 61.65) (end 170.3 81.71) (width 0.25) (layer "F.Cu") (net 4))
 (segment (start 90.2 42.045) (end 91.225 43.07) (width 0.25) (layer "F.Cu") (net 4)))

